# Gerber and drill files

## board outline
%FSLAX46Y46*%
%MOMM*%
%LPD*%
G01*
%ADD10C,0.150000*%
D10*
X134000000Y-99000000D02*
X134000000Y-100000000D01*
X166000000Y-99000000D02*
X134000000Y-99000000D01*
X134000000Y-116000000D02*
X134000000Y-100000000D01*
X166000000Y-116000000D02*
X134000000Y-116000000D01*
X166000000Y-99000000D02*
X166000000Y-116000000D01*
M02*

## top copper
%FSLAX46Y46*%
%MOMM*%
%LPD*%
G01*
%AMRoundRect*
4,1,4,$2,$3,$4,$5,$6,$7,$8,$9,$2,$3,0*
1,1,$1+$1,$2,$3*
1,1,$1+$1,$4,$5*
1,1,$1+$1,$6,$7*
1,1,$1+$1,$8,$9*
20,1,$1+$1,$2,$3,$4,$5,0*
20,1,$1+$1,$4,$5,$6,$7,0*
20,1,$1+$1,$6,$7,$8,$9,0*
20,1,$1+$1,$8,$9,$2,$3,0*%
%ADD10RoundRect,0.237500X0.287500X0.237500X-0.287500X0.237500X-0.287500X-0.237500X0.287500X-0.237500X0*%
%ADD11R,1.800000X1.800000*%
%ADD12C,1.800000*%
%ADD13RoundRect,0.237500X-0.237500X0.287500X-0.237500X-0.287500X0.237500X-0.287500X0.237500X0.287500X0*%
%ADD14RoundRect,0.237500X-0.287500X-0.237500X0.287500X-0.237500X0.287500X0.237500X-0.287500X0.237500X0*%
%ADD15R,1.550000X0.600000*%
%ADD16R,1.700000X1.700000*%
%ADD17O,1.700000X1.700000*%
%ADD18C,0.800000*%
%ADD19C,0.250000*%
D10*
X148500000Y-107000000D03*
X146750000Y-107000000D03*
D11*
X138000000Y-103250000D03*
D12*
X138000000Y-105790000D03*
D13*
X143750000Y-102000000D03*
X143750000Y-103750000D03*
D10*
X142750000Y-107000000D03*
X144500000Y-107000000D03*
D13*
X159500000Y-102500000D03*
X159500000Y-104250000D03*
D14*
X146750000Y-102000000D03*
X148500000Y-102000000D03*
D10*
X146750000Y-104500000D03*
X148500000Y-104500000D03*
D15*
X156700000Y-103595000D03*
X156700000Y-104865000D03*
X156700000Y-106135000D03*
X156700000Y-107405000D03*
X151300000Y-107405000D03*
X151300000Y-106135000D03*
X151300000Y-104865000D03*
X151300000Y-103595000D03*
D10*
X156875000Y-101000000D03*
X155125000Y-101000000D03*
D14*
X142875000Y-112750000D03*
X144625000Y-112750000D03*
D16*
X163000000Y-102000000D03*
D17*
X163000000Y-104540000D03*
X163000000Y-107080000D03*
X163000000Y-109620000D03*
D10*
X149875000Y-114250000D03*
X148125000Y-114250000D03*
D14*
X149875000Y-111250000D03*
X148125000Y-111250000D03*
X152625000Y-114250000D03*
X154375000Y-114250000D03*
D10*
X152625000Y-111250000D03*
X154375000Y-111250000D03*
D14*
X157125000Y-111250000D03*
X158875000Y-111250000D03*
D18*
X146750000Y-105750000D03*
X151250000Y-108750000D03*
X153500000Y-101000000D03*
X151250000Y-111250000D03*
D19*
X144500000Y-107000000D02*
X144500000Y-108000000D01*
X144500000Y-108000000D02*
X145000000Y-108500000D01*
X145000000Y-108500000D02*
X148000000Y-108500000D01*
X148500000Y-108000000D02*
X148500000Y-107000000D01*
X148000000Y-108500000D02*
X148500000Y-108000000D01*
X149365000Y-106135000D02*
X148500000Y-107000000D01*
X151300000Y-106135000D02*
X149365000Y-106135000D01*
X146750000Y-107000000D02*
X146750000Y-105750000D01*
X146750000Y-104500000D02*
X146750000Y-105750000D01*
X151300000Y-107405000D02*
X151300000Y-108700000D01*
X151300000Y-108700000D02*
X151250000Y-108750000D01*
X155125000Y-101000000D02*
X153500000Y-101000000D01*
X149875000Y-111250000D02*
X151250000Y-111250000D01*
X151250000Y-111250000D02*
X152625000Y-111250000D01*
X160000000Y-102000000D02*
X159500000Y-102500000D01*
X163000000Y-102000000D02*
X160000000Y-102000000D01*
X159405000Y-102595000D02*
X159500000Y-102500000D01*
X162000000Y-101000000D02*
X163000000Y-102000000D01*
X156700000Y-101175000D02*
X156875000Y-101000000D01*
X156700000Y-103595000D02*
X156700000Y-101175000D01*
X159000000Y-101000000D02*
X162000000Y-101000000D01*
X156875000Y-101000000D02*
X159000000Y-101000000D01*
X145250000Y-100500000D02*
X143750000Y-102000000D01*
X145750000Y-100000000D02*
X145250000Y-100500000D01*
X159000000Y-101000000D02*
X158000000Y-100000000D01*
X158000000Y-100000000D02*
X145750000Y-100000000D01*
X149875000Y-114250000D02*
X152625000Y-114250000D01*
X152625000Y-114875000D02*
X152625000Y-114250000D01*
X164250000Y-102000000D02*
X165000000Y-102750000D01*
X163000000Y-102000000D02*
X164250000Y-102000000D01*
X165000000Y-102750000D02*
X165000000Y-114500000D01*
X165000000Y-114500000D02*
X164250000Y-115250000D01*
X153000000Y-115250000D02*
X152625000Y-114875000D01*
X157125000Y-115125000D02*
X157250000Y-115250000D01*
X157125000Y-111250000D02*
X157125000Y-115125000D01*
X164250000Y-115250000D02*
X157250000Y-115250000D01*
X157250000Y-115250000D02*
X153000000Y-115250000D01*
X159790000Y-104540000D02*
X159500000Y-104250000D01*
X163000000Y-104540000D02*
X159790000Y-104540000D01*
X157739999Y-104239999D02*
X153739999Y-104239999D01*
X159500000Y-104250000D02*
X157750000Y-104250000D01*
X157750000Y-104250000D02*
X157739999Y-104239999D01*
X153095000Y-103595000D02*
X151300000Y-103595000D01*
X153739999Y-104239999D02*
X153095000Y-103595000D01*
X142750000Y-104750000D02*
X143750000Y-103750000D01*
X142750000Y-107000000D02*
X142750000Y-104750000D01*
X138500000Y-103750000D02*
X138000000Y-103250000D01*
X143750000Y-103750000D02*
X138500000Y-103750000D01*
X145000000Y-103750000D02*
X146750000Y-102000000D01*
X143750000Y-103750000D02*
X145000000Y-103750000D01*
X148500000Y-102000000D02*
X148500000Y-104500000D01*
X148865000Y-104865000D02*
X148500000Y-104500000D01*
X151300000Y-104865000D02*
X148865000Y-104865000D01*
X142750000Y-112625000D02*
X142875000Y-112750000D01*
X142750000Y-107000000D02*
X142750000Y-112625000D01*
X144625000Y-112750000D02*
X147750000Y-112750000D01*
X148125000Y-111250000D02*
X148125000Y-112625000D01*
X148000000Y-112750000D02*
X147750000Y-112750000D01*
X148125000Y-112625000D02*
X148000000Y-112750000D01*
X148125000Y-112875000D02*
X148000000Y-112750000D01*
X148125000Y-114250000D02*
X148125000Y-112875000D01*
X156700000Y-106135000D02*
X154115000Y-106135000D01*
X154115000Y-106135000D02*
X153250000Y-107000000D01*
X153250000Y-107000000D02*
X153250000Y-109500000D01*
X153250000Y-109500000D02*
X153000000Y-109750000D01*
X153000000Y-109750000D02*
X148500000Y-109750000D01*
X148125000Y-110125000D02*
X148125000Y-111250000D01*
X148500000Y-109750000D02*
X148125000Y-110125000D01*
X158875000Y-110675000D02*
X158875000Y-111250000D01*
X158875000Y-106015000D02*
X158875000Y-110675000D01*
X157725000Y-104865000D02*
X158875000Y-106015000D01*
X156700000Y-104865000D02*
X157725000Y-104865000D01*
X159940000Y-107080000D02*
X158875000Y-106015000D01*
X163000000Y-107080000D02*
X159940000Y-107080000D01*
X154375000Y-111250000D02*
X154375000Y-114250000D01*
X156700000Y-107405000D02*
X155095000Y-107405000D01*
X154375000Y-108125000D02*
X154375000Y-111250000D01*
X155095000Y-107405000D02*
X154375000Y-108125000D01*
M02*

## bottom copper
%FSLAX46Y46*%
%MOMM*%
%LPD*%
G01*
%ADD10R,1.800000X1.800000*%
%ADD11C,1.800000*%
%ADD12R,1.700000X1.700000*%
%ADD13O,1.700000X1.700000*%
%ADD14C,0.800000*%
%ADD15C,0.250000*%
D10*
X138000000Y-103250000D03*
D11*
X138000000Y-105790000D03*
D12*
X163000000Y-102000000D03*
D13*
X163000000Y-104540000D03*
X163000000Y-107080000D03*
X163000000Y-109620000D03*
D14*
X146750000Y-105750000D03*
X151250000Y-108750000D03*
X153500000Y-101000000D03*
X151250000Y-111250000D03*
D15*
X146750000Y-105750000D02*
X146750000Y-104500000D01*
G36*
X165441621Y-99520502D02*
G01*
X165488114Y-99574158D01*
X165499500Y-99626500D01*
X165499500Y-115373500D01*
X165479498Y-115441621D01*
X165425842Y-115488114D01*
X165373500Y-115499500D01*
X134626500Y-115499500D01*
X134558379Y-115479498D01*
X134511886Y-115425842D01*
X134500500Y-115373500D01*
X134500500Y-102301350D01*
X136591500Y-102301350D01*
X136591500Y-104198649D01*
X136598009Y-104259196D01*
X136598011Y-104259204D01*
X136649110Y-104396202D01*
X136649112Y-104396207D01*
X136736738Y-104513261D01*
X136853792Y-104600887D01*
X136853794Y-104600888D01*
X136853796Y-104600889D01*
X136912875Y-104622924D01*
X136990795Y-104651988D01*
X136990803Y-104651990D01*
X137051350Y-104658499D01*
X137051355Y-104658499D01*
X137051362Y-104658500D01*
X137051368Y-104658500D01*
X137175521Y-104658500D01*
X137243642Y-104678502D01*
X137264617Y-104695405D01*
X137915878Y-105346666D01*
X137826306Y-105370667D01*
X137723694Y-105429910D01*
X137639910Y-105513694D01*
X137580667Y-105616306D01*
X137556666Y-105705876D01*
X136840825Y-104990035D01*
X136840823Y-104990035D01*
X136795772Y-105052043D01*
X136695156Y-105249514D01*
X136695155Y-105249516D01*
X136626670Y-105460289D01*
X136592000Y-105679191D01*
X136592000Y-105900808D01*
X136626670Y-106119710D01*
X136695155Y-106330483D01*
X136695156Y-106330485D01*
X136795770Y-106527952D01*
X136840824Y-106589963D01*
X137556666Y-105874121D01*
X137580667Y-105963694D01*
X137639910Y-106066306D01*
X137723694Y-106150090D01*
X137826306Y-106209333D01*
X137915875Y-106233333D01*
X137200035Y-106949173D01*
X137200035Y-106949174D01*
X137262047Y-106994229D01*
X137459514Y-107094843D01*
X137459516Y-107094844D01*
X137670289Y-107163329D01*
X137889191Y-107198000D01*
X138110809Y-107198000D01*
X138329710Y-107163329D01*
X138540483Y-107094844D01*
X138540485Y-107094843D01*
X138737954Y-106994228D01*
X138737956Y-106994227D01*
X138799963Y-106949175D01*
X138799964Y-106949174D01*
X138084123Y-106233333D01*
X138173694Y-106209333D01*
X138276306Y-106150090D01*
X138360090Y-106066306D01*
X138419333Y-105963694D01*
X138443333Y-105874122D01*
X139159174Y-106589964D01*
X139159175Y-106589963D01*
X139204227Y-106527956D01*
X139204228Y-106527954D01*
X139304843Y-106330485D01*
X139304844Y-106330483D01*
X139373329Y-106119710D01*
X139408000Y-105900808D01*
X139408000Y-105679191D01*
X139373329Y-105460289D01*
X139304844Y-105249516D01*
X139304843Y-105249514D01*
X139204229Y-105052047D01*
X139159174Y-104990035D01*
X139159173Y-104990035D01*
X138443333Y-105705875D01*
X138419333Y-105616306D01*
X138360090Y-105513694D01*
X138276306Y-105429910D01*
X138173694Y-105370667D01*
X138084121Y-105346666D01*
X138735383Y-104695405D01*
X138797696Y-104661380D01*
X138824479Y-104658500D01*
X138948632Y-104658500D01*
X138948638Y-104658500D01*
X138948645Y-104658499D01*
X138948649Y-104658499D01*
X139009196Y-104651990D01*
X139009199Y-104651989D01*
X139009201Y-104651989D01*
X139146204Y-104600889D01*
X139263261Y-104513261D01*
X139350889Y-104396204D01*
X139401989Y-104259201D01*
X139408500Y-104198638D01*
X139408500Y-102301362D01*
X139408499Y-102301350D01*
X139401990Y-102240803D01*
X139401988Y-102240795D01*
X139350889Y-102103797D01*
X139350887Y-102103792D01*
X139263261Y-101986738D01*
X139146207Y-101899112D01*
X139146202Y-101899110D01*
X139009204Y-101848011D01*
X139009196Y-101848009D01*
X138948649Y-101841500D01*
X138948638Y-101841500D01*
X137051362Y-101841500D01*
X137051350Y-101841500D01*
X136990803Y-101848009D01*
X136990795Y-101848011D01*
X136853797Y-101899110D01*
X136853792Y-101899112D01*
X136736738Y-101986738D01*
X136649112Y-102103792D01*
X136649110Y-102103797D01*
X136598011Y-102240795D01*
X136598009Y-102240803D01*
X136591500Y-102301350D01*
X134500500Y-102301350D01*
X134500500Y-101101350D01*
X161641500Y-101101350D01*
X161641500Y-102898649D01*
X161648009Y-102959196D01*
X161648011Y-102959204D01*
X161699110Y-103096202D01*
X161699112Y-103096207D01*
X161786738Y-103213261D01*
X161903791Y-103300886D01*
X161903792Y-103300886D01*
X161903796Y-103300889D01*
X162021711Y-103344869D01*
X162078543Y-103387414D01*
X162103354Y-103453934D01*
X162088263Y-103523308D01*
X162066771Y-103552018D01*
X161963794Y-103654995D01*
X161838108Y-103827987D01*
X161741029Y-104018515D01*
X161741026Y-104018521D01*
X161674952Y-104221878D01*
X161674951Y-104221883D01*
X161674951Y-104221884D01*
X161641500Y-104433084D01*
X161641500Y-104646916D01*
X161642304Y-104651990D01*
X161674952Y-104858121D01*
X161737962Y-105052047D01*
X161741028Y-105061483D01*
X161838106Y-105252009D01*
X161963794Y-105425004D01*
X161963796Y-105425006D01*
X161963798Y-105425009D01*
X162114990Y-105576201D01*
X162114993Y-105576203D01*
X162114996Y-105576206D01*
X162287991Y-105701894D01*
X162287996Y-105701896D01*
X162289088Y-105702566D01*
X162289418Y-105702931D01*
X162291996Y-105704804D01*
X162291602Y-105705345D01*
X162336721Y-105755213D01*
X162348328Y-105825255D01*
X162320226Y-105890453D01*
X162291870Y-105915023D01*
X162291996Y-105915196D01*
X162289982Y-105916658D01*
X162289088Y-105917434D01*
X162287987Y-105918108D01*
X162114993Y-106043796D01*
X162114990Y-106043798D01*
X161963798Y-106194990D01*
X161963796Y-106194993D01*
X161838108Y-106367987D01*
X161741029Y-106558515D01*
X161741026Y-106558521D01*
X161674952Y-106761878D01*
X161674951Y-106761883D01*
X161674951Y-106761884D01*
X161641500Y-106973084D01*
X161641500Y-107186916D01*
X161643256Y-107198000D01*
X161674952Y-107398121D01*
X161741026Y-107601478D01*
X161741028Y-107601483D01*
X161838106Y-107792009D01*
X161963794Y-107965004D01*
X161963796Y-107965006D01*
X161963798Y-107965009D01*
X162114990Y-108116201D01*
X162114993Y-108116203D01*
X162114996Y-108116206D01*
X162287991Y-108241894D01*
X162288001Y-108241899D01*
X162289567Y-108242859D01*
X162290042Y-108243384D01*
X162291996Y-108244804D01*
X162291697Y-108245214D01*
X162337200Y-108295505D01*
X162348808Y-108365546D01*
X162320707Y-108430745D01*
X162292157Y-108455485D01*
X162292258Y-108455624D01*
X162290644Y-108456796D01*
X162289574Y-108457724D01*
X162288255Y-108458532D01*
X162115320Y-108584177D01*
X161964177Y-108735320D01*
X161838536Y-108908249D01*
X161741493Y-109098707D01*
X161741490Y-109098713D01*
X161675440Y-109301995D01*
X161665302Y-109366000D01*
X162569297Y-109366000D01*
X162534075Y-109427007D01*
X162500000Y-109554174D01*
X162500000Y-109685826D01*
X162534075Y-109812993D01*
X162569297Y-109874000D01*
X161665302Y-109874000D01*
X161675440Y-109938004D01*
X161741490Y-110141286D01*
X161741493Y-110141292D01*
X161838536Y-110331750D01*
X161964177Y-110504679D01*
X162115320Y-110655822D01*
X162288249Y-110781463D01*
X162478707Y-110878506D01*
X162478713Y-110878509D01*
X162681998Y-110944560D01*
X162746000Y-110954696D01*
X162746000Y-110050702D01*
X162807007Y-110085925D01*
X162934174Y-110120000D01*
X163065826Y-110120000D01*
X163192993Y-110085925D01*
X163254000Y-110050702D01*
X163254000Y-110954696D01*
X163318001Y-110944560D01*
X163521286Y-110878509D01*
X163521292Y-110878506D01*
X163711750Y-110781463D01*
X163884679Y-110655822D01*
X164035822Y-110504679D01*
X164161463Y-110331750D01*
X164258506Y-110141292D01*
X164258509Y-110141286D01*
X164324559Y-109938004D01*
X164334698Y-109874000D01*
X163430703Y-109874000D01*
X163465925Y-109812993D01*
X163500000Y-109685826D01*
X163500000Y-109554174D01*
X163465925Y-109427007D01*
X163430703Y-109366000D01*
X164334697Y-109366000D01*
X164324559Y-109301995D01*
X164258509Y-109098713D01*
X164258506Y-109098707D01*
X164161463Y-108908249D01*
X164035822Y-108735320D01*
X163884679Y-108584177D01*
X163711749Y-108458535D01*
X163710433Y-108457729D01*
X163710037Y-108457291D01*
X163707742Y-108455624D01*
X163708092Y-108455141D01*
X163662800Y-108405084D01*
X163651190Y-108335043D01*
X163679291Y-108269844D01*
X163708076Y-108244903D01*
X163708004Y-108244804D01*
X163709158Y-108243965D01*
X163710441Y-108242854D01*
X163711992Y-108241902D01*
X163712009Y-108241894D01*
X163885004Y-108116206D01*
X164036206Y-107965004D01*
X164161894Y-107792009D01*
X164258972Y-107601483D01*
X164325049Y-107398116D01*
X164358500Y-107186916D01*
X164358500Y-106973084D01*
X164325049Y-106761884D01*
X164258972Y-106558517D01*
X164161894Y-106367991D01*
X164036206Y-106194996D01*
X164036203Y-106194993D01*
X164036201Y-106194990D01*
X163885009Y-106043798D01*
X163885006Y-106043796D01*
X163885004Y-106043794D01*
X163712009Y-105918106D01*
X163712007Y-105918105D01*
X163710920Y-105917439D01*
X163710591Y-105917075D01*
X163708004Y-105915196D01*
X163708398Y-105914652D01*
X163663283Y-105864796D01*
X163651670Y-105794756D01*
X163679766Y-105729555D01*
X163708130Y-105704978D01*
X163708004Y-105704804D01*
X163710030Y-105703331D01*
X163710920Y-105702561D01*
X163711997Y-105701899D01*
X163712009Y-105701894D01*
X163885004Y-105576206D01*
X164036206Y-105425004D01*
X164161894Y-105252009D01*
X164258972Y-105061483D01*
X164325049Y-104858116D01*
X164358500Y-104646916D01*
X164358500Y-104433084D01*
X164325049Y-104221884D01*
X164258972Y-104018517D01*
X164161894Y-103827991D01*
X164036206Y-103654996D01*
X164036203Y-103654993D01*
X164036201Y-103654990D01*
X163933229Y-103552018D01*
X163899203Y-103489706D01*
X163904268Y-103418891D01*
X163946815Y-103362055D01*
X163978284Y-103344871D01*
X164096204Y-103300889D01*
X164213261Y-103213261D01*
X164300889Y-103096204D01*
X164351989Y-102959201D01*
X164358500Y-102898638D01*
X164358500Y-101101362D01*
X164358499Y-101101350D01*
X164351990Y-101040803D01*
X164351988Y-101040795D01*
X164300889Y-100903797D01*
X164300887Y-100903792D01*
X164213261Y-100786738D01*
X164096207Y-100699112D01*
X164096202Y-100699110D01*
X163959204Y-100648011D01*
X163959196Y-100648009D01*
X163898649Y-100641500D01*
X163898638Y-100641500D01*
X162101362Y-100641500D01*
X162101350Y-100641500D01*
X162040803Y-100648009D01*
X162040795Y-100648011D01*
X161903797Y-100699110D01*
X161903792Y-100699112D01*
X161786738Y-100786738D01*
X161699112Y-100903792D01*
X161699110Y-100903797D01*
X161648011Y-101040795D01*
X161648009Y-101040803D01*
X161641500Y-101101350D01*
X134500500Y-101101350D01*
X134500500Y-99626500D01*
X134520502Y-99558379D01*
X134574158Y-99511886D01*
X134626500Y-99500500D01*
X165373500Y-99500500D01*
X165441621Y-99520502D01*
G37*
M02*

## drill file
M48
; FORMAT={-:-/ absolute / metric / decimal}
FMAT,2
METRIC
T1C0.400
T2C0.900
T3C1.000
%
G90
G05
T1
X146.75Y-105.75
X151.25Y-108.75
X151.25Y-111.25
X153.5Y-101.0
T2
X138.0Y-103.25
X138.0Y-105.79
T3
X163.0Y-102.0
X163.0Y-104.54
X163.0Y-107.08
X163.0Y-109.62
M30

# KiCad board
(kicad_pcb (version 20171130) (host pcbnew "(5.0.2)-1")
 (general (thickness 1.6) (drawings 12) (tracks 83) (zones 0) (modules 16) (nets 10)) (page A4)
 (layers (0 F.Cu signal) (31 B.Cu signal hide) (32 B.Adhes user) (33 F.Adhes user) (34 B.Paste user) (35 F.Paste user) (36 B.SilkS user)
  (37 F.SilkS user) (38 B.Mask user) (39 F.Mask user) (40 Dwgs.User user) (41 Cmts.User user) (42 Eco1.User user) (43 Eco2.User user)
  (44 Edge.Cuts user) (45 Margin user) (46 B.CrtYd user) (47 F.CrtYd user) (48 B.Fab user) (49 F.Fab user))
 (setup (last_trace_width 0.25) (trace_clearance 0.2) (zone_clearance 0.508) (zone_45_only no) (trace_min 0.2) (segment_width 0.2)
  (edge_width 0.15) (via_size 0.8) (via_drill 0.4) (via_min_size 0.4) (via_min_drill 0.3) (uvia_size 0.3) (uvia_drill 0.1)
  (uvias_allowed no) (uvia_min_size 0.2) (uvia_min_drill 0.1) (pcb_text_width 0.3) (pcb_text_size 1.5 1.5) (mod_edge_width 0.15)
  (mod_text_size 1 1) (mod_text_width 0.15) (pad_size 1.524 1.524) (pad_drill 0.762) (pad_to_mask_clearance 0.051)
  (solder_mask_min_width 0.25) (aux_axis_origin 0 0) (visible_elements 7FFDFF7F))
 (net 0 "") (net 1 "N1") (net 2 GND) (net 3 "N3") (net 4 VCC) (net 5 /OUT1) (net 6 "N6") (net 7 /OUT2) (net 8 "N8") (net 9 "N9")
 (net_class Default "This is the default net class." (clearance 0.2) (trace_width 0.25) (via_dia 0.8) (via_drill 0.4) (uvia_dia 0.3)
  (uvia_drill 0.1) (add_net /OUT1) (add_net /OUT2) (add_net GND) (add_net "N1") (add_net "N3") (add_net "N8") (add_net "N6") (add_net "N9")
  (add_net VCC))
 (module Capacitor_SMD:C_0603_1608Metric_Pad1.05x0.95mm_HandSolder (layer F.Cu) (at 147.625 107 180)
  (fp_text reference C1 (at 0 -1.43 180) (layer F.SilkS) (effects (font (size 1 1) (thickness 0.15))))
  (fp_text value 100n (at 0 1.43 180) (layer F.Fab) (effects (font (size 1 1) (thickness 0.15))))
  (pad 1 smd roundrect (at -0.875 0 180) (size 1.05 0.95) (layers F.Cu F.Paste F.Mask) (roundrect_rratio 0.25) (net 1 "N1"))
  (pad 2 smd roundrect (at 0.875 0 180) (size 1.05 0.95) (layers F.Cu F.Paste F.Mask) (roundrect_rratio 0.25) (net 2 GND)))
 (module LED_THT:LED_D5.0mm (layer F.Cu) (at 138 103.25 270)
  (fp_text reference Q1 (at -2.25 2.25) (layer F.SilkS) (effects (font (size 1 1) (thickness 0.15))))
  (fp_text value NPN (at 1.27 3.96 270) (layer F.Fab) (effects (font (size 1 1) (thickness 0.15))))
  (pad 1 thru_hole rect (at 0 0 270) (size 1.8 1.8) (drill 0.9) (layers *.Cu *.Mask) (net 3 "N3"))
  (pad 2 thru_hole circle (at 2.54 0 270) (size 1.8 1.8) (drill 0.9) (layers *.Cu *.Mask) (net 2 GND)))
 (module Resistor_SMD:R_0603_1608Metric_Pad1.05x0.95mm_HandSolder (layer F.Cu) (at 143.75 102.875 270)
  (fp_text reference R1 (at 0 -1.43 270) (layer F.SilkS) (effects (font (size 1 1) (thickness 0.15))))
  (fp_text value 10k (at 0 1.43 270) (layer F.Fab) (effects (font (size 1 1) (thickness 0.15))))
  (pad 1 smd roundrect (at -0.875 0 270) (size 1.05 0.95) (layers F.Cu F.Paste F.Mask) (roundrect_rratio 0.25) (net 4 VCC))
  (pad 2 smd roundrect (at 0.875 0 270) (size 1.05 0.95) (layers F.Cu F.Paste F.Mask) (roundrect_rratio 0.25) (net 3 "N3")))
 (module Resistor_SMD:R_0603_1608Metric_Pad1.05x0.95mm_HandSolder (layer F.Cu) (at 143.625 107 180)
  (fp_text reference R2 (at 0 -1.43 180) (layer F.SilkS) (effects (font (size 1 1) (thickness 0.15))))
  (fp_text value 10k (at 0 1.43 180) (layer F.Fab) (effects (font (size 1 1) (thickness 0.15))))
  (pad 2 smd roundrect (at 0.875 0 180) (size 1.05 0.95) (layers F.Cu F.Paste F.Mask) (roundrect_rratio 0.25) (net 3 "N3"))
  (pad 1 smd roundrect (at -0.875 0 180) (size 1.05 0.95) (layers F.Cu F.Paste F.Mask) (roundrect_rratio 0.25) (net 1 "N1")))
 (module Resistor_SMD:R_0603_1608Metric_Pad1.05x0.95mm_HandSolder (layer F.Cu) (at 159.5 103.375 270)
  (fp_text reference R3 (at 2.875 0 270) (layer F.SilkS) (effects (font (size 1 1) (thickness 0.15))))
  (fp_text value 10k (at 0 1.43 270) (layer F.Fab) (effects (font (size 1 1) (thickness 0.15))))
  (pad 1 smd roundrect (at -0.875 0 270) (size 1.05 0.95) (layers F.Cu F.Paste F.Mask) (roundrect_rratio 0.25) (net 4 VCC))
  (pad 2 smd roundrect (at 0.875 0 270) (size 1.05 0.95) (layers F.Cu F.Paste F.Mask) (roundrect_rratio 0.25) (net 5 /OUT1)))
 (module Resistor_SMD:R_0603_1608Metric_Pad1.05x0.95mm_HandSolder (layer F.Cu) (at 147.625 102)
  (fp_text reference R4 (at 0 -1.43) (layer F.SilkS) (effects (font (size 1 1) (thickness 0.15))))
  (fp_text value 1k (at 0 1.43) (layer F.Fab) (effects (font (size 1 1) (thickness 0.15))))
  (pad 1 smd roundrect (at -0.875 0) (size 1.05 0.95) (layers F.Cu F.Paste F.Mask) (roundrect_rratio 0.25) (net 3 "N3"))
  (pad 2 smd roundrect (at 0.875 0) (size 1.05 0.95) (layers F.Cu F.Paste F.Mask) (roundrect_rratio 0.25) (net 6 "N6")))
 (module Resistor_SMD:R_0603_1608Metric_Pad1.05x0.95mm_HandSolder (layer F.Cu) (at 147.625 104.5 180)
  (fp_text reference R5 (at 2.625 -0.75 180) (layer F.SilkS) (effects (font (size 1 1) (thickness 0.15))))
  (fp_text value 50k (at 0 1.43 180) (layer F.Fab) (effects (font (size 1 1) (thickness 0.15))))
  (pad 2 smd roundrect (at 0.875 0 180) (size 1.05 0.95) (layers F.Cu F.Paste F.Mask) (roundrect_rratio 0.25) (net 2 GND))
  (pad 1 smd roundrect (at -0.875 0 180) (size 1.05 0.95) (layers F.Cu F.Paste F.Mask) (roundrect_rratio 0.25) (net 6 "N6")))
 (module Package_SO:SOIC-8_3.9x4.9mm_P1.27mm (layer F.Cu) (at 154 105.5)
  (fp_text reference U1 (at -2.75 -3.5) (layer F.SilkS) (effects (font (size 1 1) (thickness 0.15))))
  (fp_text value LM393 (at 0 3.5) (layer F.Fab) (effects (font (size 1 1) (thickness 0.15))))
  (pad 8 smd rect (at 2.7 -1.905) (size 1.55 0.6) (layers F.Cu F.Paste F.Mask) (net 4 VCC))
  (pad 7 smd rect (at 2.7 -0.635) (size 1.55 0.6) (layers F.Cu F.Paste F.Mask) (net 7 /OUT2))
  (pad 6 smd rect (at 2.7 0.635) (size 1.55 0.6) (layers F.Cu F.Paste F.Mask) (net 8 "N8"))
  (pad 5 smd rect (at 2.7 1.905) (size 1.55 0.6) (layers F.Cu F.Paste F.Mask) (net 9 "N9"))
  (pad 4 smd rect (at -2.7 1.905) (size 1.55 0.6) (layers F.Cu F.Paste F.Mask) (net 2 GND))
  (pad 3 smd rect (at -2.7 0.635) (size 1.55 0.6) (layers F.Cu F.Paste F.Mask) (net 1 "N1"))
  (pad 2 smd rect (at -2.7 -0.635) (size 1.55 0.6) (layers F.Cu F.Paste F.Mask) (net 6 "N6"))
  (pad 1 smd rect (at -2.7 -1.905) (size 1.55 0.6) (layers F.Cu F.Paste F.Mask) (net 5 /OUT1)))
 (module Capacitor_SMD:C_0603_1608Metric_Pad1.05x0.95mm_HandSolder (layer F.Cu) (at 156 101 180)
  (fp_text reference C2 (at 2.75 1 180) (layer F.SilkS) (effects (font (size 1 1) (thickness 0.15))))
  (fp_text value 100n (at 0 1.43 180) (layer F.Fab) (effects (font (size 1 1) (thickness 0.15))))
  (pad 1 smd roundrect (at -0.875 0 180) (size 1.05 0.95) (layers F.Cu F.Paste F.Mask) (roundrect_rratio 0.25) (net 4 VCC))
  (pad 2 smd roundrect (at 0.875 0 180) (size 1.05 0.95) (layers F.Cu F.Paste F.Mask) (roundrect_rratio 0.25) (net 2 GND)))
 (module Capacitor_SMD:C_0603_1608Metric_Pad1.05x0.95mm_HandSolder (layer F.Cu) (at 143.75 112.75)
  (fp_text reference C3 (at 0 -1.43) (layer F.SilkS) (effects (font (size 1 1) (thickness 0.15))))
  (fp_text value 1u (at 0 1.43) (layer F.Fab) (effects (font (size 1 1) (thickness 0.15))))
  (pad 1 smd roundrect (at -0.875 0) (size 1.05 0.95) (layers F.Cu F.Paste F.Mask) (roundrect_rratio 0.25) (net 3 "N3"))
  (pad 2 smd roundrect (at 0.875 0) (size 1.05 0.95) (layers F.Cu F.Paste F.Mask) (roundrect_rratio 0.25) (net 8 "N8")))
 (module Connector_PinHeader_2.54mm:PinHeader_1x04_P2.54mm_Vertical (layer F.Cu) (at 163 102)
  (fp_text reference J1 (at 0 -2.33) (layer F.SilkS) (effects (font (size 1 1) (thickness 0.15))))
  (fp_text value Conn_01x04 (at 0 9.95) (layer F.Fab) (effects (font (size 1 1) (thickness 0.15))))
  (pad 1 thru_hole rect (at 0 0) (size 1.7 1.7) (drill 1) (layers *.Cu *.Mask) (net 4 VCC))
  (pad 2 thru_hole oval (at 0 2.54) (size 1.7 1.7) (drill 1) (layers *.Cu *.Mask) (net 5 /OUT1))
  (pad 3 thru_hole oval (at 0 5.08) (size 1.7 1.7) (drill 1) (layers *.Cu *.Mask) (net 7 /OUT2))
  (pad 4 thru_hole oval (at 0 7.62) (size 1.7 1.7) (drill 1) (layers *.Cu *.Mask) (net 2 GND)))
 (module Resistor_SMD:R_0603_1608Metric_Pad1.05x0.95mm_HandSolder (layer F.Cu) (at 149 114.25 180)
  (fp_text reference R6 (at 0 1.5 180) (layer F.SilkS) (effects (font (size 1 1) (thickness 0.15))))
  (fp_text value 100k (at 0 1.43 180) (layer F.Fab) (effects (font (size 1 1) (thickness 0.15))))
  (pad 1 smd roundrect (at -0.875 0 180) (size 1.05 0.95) (layers F.Cu F.Paste F.Mask) (roundrect_rratio 0.25) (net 4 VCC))
  (pad 2 smd roundrect (at 0.875 0 180) (size 1.05 0.95) (layers F.Cu F.Paste F.Mask) (roundrect_rratio 0.25) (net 8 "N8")))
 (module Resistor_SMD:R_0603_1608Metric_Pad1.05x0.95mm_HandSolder (layer F.Cu) (at 149 111.25)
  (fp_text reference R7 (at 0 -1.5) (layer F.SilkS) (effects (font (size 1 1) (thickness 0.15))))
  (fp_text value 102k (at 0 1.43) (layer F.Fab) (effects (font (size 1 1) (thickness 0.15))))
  (pad 2 smd roundrect (at 0.875 0) (size 1.05 0.95) (layers F.Cu F.Paste F.Mask) (roundrect_rratio 0.25) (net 2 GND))
  (pad 1 smd roundrect (at -0.875 0) (size 1.05 0.95) (layers F.Cu F.Paste F.Mask) (roundrect_rratio 0.25) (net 8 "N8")))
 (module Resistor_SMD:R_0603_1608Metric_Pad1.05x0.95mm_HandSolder (layer F.Cu) (at 153.5 114.25)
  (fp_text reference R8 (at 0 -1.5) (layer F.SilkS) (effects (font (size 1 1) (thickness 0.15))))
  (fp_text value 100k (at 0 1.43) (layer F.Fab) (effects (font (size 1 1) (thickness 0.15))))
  (pad 1 smd roundrect (at -0.875 0) (size 1.05 0.95) (layers F.Cu F.Paste F.Mask) (roundrect_rratio 0.25) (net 4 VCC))
  (pad 2 smd roundrect (at 0.875 0) (size 1.05 0.95) (layers F.Cu F.Paste F.Mask) (roundrect_rratio 0.25) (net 9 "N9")))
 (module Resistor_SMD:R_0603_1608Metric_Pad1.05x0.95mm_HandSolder (layer F.Cu) (at 153.5 111.25 180)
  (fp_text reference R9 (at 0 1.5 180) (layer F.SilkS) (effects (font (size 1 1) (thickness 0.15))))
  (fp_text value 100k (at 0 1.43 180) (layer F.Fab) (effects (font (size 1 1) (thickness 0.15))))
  (pad 2 smd roundrect (at 0.875 0 180) (size 1.05 0.95) (layers F.Cu F.Paste F.Mask) (roundrect_rratio 0.25) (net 2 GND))
  (pad 1 smd roundrect (at -0.875 0 180) (size 1.05 0.95) (layers F.Cu F.Paste F.Mask) (roundrect_rratio 0.25) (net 9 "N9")))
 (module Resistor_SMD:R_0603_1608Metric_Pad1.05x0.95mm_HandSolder (layer F.Cu) (at 158 111.25)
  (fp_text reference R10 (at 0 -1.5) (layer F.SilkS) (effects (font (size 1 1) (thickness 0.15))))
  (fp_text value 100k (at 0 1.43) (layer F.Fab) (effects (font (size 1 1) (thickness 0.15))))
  (pad 1 smd roundrect (at -0.875 0) (size 1.05 0.95) (layers F.Cu F.Paste F.Mask) (roundrect_rratio 0.25) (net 4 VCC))
  (pad 2 smd roundrect (at 0.875 0) (size 1.05 0.95) (layers F.Cu F.Paste F.Mask) (roundrect_rratio 0.25) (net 7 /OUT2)))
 (gr_line (start 134 99) (end 134 100) (layer Edge.Cuts) (width 0.15))
 (gr_line (start 166 99) (end 134 99) (layer Edge.Cuts) (width 0.15))
 (gr_line (start 134 116) (end 134 100) (layer Edge.Cuts) (width 0.15))
 (gr_line (start 166 116) (end 134 116) (layer Edge.Cuts) (width 0.15))
 (gr_line (start 166 99) (end 166 116) (layer Edge.Cuts) (width 0.15))
 (segment (start 144.5 107) (end 144.5 108) (width 0.25) (layer F.Cu) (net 1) (status 10))
 (segment (start 144.5 108) (end 145 108.5) (width 0.25) (layer F.Cu) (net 1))
 (segment (start 145 108.5) (end 148 108.5) (width 0.25) (layer F.Cu) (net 1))
 (segment (start 148.5 108) (end 148.5 107) (width 0.25) (layer F.Cu) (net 1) (status 20))
 (segment (start 148 108.5) (end 148.5 108) (width 0.25) (layer F.Cu) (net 1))
 (segment (start 149.365 106.135) (end 148.5 107) (width 0.25) (layer F.Cu) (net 1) (status 20))
 (segment (start 151.3 106.135) (end 149.365 106.135) (width 0.25) (layer F.Cu) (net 1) (status 10))
 (via (at 146.75 105.75) (size 0.8) (drill 0.4) (layers F.Cu B.Cu) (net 2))
 (segment (start 146.75 107) (end 146.75 105.75) (width 0.25) (layer F.Cu) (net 2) (status 10))
 (segment (start 146.75 105.75) (end 146.75 104.5) (width 0.25) (layer B.Cu) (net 2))
 (segment (start 146.75 104.5) (end 146.75 105.75) (width 0.25) (layer F.Cu) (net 2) (status 10))
 (via (at 151.25 108.75) (size 0.8) (drill 0.4) (layers F.Cu B.Cu) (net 2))
 (segment (start 151.3 107.405) (end 151.3 108.7) (width 0.25) (layer F.Cu) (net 2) (status 10))
 (segment (start 151.3 108.7) (end 151.25 108.75) (width 0.25) (layer F.Cu) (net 2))
 (via (at 153.5 101) (size 0.8) (drill 0.4) (layers F.Cu B.Cu) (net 2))
 (segment (start 155.125 101) (end 153.5 101) (width 0.25) (layer F.Cu) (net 2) (status 10))
 (segment (start 149.875 111.25) (end 151.25 111.25) (width 0.25) (layer F.Cu) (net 2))
 (segment (start 151.25 111.25) (end 152.625 111.25) (width 0.25) (layer F.Cu) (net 2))
 (via (at 151.25 111.25) (size 0.8) (drill 0.4) (layers F.Cu B.Cu) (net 2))
 (segment (start 160 102) (end 159.5 102.5) (width 0.25) (layer F.Cu) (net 4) (status 20))
 (segment (start 163 102) (end 160 102) (width 0.25) (layer F.Cu) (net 4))
 (segment (start 159.405 102.595) (end 159.5 102.5) (width 0.25) (layer F.Cu) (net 4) (status 30))
 (segment (start 162 101) (end 163 102) (width 0.25) (layer F.Cu) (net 4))
 (segment (start 156.7 101.175) (end 156.875 101) (width 0.25) (layer F.Cu) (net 4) (status 30))
 (segment (start 156.7 103.595) (end 156.7 101.175) (width 0.25) (layer F.Cu) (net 4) (status 30))
 (segment (start 159 101) (end 162 101) (width 0.25) (layer F.Cu) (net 4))
 (segment (start 156.875 101) (end 159 101) (width 0.25) (layer F.Cu) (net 4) (status 10))
 (segment (start 145.25 100.5) (end 143.75 102) (width 0.25) (layer F.Cu) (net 4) (status 20))
 (segment (start 145.75 100) (end 145.25 100.5) (width 0.25) (layer F.Cu) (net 4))
 (segment (start 159 101) (end 158 100) (width 0.25) (layer F.Cu) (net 4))
 (segment (start 158 100) (end 145.75 100) (width 0.25) (layer F.Cu) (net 4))
 (segment (start 149.875 114.25) (end 152.625 114.25) (width 0.25) (layer F.Cu) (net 4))
 (segment (start 152.625 114.875) (end 152.625 114.25) (width 0.25) (layer F.Cu) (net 4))
 (segment (start 164.25 102) (end 165 102.75) (width 0.25) (layer F.Cu) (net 4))
 (segment (start 163 102) (end 164.25 102) (width 0.25) (layer F.Cu) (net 4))
 (segment (start 165 102.75) (end 165 114.5) (width 0.25) (layer F.Cu) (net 4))
 (segment (start 165 114.5) (end 164.25 115.25) (width 0.25) (layer F.Cu) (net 4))
 (segment (start 153 115.25) (end 152.625 114.875) (width 0.25) (layer F.Cu) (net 4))
 (segment (start 157.125 115.125) (end 157.25 115.25) (width 0.25) (layer F.Cu) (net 4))
 (segment (start 157.125 111.25) (end 157.125 115.125) (width 0.25) (layer F.Cu) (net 4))
 (segment (start 164.25 115.25) (end 157.25 115.25) (width 0.25) (layer F.Cu) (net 4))
 (segment (start 157.25 115.25) (end 153 115.25) (width 0.25) (layer F.Cu) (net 4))
 (segment (start 159.79 104.54) (end 159.5 104.25) (width 0.25) (layer F.Cu) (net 5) (status 30))
 (segment (start 163 104.54) (end 159.79 104.54) (width 0.25) (layer F.Cu) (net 5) (status 20))
 (segment (start 157.739999 104.239999) (end 153.739999 104.239999) (width 0.25) (layer F.Cu) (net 5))
 (segment (start 159.5 104.25) (end 157.75 104.25) (width 0.25) (layer F.Cu) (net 5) (status 10))
 (segment (start 157.75 104.25) (end 157.739999 104.239999) (width 0.25) (layer F.Cu) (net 5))
 (segment (start 153.095 103.595) (end 151.3 103.595) (width 0.25) (layer F.Cu) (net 5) (status 20))
 (segment (start 153.739999 104.239999) (end 153.095 103.595) (width 0.25) (layer F.Cu) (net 5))
 (segment (start 142.75 104.75) (end 143.75 103.75) (width 0.25) (layer F.Cu) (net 3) (status 20))
 (segment (start 142.75 107) (end 142.75 104.75) (width 0.25) (layer F.Cu) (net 3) (status 10))
 (segment (start 138.5 103.75) (end 138 103.25) (width 0.25) (layer F.Cu) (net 3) (status 30))
 (segment (start 143.75 103.75) (end 138.5 103.75) (width 0.25) (layer F.Cu) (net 3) (status 30))
 (segment (start 145 103.75) (end 146.75 102) (width 0.25) (layer F.Cu) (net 3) (status 20))
 (segment (start 143.75 103.75) (end 145 103.75) (width 0.25) (layer F.Cu) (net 3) (status 10))
 (segment (start 148.5 102) (end 148.5 104.5) (width 0.25) (layer F.Cu) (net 6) (status 30))
 (segment (start 148.865 104.865) (end 148.5 104.5) (width 0.25) (layer F.Cu) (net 6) (status 30))
 (segment (start 151.3 104.865) (end 148.865 104.865) (width 0.25) (layer F.Cu) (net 6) (status 30))
 (segment (start 142.75 112.625) (end 142.875 112.75) (width 0.25) (layer F.Cu) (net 3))
 (segment (start 142.75 107) (end 142.75 112.625) (width 0.25) (layer F.Cu) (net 3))
 (segment (start 144.625 112.75) (end 147.75 112.75) (width 0.25) (layer F.Cu) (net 8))
 (segment (start 148.125 111.25) (end 148.125 112.625) (width 0.25) (layer F.Cu) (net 8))
 (segment (start 148 112.75) (end 147.75 112.75) (width 0.25) (layer F.Cu) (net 8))
 (segment (start 148.125 112.625) (end 148 112.75) (width 0.25) (layer F.Cu) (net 8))
 (segment (start 148.125 112.875) (end 148 112.75) (width 0.25) (layer F.Cu) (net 8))
 (segment (start 148.125 114.25) (end 148.125 112.875) (width 0.25) (layer F.Cu) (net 8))
 (segment (start 156.7 106.135) (end 154.115 106.135) (width 0.25) (layer F.Cu) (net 8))
 (segment (start 154.115 106.135) (end 153.25 107) (width 0.25) (layer F.Cu) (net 8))
 (segment (start 153.25 107) (end 153.25 109.5) (width 0.25) (layer F.Cu) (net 8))
 (segment (start 153.25 109.5) (end 153 109.75) (width 0.25) (layer F.Cu) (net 8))
 (segment (start 153 109.75) (end 148.5 109.75) (width 0.25) (layer F.Cu) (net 8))
 (segment (start 148.125 110.125) (end 148.125 111.25) (width 0.25) (layer F.Cu) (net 8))
 (segment (start 148.5 109.75) (end 148.125 110.125) (width 0.25) (layer F.Cu) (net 8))
 (segment (start 158.875 110.675) (end 158.875 111.25) (width 0.25) (layer F.Cu) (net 7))
 (segment (start 158.875 106.015) (end 158.875 110.675) (width 0.25) (layer F.Cu) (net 7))
 (segment (start 157.725 104.865) (end 158.875 106.015) (width 0.25) (layer F.Cu) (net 7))
 (segment (start 156.7 104.865) (end 157.725 104.865) (width 0.25) (layer F.Cu) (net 7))
 (segment (start 159.94 107.08) (end 158.875 106.015) (width 0.25) (layer F.Cu) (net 7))
 (segment (start 163 107.08) (end 159.94 107.08) (width 0.25) (layer F.Cu) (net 7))
 (segment (start 154.375 111.25) (end 154.375 114.25) (width 0.25) (layer F.Cu) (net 9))
 (segment (start 156.7 107.405) (end 155.095 107.405) (width 0.25) (layer F.Cu) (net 9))
 (segment (start 154.375 108.125) (end 154.375 111.25) (width 0.25) (layer F.Cu) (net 9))
 (segment (start 155.095 107.405) (end 154.375 108.125) (width 0.25) (layer F.Cu) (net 9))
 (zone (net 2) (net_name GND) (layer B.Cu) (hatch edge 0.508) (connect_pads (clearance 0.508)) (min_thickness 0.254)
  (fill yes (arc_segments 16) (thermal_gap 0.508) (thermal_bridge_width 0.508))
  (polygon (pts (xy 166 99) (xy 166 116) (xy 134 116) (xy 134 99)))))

